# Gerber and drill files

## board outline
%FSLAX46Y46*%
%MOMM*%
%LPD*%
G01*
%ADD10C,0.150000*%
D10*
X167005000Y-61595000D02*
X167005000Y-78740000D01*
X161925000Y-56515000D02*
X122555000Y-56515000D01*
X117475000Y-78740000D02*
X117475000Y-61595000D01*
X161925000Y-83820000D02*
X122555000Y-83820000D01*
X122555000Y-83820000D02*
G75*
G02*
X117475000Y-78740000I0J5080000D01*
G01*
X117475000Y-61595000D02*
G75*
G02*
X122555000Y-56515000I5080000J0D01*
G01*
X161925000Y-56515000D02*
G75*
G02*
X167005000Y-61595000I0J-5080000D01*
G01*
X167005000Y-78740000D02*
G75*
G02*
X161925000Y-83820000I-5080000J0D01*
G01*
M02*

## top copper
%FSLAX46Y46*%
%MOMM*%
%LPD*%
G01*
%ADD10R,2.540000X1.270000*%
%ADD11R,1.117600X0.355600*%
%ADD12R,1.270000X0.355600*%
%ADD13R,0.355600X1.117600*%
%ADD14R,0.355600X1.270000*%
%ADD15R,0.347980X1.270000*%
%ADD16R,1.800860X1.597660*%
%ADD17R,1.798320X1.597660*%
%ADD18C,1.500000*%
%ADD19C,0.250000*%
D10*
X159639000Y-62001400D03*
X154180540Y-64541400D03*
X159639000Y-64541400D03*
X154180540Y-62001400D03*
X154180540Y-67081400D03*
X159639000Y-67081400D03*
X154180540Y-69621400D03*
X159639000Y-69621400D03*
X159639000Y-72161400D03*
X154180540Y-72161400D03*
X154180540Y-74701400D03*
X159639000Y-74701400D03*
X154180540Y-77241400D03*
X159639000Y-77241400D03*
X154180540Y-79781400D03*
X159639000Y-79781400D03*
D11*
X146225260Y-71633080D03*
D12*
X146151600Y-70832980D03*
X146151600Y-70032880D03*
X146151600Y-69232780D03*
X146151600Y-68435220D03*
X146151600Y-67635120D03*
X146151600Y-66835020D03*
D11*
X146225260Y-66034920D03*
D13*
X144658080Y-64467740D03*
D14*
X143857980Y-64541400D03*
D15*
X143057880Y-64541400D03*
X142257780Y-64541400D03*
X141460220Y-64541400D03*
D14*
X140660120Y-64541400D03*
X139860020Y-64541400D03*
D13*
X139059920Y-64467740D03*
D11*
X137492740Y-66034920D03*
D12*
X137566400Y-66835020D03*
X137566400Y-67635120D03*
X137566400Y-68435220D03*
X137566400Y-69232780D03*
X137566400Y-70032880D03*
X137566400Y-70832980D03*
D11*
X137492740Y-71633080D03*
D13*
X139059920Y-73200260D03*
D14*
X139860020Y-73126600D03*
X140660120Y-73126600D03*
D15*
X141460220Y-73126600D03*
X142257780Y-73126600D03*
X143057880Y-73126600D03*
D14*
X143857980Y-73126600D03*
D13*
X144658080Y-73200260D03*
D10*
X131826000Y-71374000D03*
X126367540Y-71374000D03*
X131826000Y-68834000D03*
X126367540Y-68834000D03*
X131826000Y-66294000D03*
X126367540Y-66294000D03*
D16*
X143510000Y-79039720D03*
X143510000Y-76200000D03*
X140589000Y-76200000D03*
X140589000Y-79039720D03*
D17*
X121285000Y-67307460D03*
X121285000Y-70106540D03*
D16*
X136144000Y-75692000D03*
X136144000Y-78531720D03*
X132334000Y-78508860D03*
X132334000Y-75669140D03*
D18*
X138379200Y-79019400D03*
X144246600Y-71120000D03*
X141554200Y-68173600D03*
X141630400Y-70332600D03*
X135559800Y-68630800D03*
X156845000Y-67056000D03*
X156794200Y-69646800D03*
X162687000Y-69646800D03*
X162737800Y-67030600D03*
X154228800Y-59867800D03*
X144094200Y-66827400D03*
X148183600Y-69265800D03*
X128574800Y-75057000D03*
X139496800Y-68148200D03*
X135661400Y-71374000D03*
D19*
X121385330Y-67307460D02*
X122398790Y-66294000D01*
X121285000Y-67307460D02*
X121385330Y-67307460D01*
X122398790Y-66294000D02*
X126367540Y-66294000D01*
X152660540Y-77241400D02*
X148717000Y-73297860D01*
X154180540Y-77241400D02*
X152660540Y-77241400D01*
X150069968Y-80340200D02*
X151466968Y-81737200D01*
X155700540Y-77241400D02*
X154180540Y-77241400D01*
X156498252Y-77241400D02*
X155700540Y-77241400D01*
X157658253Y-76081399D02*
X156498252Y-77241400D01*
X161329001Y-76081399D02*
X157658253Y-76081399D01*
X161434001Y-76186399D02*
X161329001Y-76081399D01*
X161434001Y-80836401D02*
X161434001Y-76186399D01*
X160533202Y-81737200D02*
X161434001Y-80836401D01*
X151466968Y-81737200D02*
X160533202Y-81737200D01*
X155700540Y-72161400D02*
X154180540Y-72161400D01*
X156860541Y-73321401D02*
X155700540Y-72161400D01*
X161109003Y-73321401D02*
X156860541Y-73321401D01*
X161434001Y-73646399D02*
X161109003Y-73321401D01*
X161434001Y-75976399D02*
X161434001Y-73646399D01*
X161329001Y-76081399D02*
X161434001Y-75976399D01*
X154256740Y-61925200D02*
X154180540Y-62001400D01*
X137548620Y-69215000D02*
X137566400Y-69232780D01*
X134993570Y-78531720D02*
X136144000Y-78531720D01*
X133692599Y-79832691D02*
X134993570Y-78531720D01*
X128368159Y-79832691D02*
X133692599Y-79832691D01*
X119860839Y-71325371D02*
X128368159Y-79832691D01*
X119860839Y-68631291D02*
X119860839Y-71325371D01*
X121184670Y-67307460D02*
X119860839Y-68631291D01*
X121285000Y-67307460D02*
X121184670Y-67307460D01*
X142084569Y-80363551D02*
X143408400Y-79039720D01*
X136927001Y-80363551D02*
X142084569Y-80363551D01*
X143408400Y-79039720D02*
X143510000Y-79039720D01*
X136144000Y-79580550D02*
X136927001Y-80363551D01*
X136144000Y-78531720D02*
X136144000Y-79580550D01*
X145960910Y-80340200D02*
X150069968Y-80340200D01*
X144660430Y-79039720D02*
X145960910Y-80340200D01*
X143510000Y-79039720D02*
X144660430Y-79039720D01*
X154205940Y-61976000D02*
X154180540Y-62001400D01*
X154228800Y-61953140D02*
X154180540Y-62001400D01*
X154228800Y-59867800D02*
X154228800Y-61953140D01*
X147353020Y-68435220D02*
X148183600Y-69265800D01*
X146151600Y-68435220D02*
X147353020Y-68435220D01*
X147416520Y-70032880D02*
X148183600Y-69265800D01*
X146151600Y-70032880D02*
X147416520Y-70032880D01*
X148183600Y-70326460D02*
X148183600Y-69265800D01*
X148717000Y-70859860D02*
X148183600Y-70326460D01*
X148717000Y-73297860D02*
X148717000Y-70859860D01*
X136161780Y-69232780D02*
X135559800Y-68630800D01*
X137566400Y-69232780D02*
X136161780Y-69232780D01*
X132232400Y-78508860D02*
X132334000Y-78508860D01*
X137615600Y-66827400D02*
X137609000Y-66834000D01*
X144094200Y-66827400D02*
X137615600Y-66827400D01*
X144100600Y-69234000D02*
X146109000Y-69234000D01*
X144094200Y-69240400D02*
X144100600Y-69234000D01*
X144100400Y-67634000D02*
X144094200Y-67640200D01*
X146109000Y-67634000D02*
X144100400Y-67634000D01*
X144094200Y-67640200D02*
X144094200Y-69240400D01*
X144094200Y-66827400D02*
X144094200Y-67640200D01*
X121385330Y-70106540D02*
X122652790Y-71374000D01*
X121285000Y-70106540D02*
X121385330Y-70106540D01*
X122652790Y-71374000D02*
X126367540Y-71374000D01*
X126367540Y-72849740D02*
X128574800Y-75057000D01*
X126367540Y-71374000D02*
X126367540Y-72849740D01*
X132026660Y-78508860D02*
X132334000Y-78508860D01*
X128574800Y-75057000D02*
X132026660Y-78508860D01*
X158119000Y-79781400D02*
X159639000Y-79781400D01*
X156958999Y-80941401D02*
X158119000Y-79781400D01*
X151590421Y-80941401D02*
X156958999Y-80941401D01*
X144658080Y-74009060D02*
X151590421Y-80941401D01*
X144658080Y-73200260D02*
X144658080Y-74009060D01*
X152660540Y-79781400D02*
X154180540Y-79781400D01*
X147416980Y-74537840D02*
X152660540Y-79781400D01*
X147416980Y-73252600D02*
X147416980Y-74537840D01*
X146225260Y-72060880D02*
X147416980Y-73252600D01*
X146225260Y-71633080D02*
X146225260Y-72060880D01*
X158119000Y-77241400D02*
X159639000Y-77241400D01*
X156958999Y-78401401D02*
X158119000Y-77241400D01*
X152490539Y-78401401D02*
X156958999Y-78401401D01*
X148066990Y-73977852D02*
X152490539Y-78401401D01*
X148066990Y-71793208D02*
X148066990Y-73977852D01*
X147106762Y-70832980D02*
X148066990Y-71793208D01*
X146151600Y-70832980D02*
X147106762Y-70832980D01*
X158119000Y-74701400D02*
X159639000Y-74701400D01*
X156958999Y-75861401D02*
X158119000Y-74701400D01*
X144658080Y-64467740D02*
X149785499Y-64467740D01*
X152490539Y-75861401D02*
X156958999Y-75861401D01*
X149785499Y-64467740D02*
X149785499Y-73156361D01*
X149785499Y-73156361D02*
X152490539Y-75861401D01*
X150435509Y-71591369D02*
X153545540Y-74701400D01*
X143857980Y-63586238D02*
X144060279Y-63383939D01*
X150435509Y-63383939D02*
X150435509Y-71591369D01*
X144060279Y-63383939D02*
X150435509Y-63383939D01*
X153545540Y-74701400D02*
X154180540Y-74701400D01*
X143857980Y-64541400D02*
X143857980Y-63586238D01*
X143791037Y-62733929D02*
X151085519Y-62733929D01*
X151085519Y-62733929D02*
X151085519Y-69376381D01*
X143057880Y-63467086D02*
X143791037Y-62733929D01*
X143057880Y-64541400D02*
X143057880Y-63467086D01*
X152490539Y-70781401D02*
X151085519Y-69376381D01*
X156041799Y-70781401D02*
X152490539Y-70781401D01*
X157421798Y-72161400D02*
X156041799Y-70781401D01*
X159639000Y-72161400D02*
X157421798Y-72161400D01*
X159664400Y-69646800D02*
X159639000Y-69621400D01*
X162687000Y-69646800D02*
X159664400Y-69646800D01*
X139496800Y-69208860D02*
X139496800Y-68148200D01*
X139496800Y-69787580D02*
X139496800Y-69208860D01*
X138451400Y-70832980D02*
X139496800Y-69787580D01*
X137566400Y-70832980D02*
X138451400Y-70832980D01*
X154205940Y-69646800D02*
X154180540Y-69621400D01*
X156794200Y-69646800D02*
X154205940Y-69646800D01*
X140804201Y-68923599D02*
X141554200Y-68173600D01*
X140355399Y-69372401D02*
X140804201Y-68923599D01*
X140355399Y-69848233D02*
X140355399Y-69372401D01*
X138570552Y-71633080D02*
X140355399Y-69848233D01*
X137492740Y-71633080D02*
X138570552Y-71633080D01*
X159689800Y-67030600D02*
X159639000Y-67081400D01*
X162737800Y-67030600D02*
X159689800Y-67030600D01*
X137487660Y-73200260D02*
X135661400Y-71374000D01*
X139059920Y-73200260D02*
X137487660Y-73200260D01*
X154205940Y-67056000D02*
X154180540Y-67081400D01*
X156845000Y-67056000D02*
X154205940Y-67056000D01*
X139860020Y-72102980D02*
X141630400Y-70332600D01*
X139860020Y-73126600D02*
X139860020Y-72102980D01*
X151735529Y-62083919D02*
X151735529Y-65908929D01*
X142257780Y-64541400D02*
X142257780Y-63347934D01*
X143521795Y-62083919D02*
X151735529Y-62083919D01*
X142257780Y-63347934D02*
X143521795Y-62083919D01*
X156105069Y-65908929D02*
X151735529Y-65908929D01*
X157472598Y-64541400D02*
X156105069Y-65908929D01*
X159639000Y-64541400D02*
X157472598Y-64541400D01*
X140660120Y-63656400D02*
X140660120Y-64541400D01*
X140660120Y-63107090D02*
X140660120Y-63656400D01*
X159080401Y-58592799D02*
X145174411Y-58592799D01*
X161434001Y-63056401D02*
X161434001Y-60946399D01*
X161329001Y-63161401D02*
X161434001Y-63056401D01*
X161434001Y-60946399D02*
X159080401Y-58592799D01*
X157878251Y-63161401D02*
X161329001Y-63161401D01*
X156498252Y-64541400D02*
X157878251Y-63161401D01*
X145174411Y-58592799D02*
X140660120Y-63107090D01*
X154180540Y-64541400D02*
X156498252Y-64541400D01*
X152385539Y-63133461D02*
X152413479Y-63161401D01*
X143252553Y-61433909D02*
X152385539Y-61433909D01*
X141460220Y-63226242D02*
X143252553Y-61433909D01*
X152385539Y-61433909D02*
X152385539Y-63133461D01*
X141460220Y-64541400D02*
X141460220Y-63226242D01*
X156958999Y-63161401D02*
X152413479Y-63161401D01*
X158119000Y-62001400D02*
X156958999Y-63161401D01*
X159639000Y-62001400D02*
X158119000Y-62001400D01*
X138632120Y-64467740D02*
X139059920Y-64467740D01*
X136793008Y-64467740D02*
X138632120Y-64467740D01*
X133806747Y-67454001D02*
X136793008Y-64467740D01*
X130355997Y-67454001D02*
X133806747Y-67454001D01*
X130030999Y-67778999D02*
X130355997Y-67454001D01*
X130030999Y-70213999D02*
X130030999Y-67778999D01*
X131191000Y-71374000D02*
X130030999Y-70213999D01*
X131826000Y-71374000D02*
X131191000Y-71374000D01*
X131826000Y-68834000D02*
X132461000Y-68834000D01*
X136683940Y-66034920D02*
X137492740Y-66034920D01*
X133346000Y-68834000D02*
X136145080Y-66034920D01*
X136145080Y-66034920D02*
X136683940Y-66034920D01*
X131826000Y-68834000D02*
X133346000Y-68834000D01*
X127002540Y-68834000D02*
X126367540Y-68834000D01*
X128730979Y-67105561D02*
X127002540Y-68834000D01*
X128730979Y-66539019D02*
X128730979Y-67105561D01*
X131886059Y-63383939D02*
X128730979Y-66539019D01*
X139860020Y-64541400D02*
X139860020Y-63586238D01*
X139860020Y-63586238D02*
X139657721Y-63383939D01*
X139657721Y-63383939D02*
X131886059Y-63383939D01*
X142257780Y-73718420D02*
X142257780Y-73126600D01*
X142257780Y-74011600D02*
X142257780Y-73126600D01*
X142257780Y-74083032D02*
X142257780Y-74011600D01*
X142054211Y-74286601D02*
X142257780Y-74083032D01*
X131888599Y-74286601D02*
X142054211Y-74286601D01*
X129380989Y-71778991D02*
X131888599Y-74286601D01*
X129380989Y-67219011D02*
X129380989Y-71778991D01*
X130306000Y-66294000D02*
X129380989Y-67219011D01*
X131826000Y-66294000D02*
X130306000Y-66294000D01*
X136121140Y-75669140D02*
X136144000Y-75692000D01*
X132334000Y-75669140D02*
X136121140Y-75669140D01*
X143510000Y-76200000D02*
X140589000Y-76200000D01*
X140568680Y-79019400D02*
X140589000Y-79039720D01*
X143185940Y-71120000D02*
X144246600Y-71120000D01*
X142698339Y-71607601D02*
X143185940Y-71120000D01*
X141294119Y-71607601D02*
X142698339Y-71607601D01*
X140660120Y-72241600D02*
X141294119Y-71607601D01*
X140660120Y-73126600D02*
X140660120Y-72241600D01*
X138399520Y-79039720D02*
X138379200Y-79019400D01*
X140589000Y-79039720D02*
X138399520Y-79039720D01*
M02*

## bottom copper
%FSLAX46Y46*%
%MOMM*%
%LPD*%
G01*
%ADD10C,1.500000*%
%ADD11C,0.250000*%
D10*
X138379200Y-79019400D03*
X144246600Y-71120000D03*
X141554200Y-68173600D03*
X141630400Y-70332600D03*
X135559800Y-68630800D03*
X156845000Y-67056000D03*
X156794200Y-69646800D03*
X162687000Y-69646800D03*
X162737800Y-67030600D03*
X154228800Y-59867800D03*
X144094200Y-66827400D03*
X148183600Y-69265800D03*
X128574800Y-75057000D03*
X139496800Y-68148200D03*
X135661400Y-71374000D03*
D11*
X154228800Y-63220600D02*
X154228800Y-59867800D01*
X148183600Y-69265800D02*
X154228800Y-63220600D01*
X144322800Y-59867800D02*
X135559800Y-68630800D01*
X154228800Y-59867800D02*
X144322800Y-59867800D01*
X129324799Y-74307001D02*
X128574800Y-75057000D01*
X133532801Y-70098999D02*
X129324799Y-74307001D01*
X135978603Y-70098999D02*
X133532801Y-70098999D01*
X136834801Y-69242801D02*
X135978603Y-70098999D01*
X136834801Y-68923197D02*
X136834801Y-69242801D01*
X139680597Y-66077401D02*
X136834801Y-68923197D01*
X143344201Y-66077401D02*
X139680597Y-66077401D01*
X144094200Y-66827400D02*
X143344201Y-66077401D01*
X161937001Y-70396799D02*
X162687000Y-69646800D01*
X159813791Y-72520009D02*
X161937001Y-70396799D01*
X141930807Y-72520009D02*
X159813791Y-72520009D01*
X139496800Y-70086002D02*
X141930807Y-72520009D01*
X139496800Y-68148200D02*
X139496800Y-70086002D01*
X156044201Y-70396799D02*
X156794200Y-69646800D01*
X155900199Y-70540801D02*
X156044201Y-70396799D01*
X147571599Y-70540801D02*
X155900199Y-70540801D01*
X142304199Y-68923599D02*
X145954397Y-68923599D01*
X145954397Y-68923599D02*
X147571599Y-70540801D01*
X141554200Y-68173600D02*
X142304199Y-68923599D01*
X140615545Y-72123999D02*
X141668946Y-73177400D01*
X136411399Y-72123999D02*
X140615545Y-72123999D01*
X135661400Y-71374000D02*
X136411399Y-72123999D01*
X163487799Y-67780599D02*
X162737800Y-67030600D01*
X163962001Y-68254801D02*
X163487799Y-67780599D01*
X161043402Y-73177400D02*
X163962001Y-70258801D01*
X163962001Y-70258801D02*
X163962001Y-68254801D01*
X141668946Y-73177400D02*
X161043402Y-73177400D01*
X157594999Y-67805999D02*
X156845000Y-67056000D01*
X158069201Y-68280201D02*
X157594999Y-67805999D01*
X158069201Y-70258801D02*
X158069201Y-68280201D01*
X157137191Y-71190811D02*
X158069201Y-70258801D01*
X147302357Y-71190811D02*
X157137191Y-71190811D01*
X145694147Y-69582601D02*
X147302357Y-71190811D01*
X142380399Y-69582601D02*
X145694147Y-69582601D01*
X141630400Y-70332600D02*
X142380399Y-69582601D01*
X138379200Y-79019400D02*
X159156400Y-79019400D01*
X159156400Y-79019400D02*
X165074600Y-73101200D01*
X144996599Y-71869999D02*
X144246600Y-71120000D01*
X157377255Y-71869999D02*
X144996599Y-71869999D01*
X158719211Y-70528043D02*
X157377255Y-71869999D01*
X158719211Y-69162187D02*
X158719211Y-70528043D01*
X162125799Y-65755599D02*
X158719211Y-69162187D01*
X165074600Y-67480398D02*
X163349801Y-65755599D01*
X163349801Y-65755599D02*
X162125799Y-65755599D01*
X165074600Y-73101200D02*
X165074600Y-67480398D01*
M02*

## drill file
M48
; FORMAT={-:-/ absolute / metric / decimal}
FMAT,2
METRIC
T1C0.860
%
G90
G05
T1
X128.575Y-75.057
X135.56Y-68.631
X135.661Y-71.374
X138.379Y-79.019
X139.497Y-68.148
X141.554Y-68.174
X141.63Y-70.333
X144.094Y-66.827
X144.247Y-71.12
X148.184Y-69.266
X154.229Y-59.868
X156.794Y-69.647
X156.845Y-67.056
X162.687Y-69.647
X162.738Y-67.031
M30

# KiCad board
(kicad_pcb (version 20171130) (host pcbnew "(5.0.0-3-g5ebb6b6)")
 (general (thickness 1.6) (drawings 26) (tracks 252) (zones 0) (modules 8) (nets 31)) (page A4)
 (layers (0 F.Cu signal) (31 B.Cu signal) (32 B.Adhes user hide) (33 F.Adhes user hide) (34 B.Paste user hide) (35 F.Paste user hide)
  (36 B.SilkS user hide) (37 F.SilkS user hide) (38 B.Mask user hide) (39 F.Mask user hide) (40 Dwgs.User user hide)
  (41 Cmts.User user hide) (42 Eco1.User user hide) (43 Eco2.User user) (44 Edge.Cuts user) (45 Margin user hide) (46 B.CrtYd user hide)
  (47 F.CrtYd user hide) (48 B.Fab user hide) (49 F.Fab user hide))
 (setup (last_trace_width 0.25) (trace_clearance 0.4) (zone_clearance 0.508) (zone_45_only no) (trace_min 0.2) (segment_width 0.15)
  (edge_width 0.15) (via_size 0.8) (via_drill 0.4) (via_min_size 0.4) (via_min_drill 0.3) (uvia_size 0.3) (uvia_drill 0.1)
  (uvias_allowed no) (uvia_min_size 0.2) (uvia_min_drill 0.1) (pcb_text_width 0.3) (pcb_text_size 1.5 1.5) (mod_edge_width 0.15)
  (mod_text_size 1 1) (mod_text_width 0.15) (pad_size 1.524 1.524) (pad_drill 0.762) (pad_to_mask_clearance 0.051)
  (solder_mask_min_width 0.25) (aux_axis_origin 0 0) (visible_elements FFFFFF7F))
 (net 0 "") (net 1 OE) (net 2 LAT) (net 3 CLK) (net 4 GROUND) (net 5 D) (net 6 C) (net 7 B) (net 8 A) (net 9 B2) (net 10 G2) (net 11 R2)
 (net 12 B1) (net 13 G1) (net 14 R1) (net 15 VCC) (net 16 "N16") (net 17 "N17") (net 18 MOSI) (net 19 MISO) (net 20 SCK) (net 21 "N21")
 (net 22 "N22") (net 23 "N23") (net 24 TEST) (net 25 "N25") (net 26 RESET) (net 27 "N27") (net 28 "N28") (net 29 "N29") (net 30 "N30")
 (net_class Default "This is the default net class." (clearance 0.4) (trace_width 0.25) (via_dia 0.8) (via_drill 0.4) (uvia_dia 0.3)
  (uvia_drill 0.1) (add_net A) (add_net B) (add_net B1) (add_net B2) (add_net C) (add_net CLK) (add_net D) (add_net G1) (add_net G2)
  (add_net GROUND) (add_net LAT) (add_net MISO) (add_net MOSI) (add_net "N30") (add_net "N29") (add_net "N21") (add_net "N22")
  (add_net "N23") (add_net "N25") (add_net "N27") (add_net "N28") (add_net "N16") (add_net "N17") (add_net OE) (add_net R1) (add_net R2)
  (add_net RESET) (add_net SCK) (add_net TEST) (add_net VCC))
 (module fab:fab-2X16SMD (layer F.Cu) (at 157.099 77.2414 180)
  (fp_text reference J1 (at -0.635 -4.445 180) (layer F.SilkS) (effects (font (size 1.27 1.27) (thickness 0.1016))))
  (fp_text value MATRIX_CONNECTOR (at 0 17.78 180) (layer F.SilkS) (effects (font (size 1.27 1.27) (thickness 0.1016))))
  (pad 15 smd rect (at -2.54 15.24 180) (size 2.54 1.27) (layers F.Cu F.Paste F.Mask) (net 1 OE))
  (pad 14 smd rect (at 2.91846 12.7 180) (size 2.54 1.27) (layers F.Cu F.Paste F.Mask) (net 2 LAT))
  (pad 13 smd rect (at -2.54 12.7 180) (size 2.54 1.27) (layers F.Cu F.Paste F.Mask) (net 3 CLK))
  (pad 16 smd rect (at 2.91846 15.24 180) (size 2.54 1.27) (layers F.Cu F.Paste F.Mask) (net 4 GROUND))
  (pad 12 smd rect (at 2.91846 10.16 180) (size 2.54 1.27) (layers F.Cu F.Paste F.Mask) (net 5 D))
  (pad 11 smd rect (at -2.54 10.16 180) (size 2.54 1.27) (layers F.Cu F.Paste F.Mask) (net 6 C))
  (pad 10 smd rect (at 2.91846 7.62 180) (size 2.54 1.27) (layers F.Cu F.Paste F.Mask) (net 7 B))
  (pad 9 smd rect (at -2.54 7.62 180) (size 2.54 1.27) (layers F.Cu F.Paste F.Mask) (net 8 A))
  (pad 7 smd rect (at -2.54 5.08 180) (size 2.54 1.27) (layers F.Cu F.Paste F.Mask) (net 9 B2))
  (pad 8 smd rect (at 2.91846 5.08 180) (size 2.54 1.27) (layers F.Cu F.Paste F.Mask) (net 4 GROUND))
  (pad 6 smd rect (at 2.91846 2.54 180) (size 2.54 1.27) (layers F.Cu F.Paste F.Mask) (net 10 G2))
  (pad 5 smd rect (at -2.54 2.54 180) (size 2.54 1.27) (layers F.Cu F.Paste F.Mask) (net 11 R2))
  (pad 4 smd rect (at 2.91846 0 180) (size 2.54 1.27) (layers F.Cu F.Paste F.Mask) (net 4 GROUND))
  (pad 3 smd rect (at -2.54 0 180) (size 2.54 1.27) (layers F.Cu F.Paste F.Mask) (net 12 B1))
  (pad 2 smd rect (at 2.91846 -2.54 180) (size 2.54 1.27) (layers F.Cu F.Paste F.Mask) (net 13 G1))
  (pad 1 smd rect (at -2.54 -2.54 180) (size 2.54 1.27) (layers F.Cu F.Paste F.Mask) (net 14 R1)))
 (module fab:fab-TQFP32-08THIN (layer F.Cu) (at 141.859 68.834 180)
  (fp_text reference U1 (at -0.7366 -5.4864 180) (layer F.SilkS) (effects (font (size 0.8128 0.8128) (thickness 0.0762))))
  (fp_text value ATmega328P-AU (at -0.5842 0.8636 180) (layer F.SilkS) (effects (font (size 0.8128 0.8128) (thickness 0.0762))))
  (pad 1 smd rect (at -4.36626 -2.79908 180) (size 1.1176 0.3556) (layers F.Cu F.Paste F.Mask) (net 13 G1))
  (pad 2 smd rect (at -4.2926 -1.99898 180) (size 1.27 0.3556) (layers F.Cu F.Paste F.Mask) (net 12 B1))
  (pad 3 smd rect (at -4.2926 -1.19888 180) (size 1.27 0.3556) (layers F.Cu F.Paste F.Mask) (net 4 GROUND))
  (pad 4 smd rect (at -4.2926 -0.39878 180) (size 1.27 0.3556) (layers F.Cu F.Paste F.Mask) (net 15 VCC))
  (pad 5 smd rect (at -4.2926 0.39878 180) (size 1.27 0.3556) (layers F.Cu F.Paste F.Mask) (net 4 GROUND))
  (pad 6 smd rect (at -4.2926 1.19888 180) (size 1.27 0.3556) (layers F.Cu F.Paste F.Mask) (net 15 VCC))
  (pad 7 smd rect (at -4.2926 1.99898 180) (size 1.27 0.3556) (layers F.Cu F.Paste F.Mask) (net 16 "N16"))
  (pad 8 smd rect (at -4.36626 2.79908 180) (size 1.1176 0.3556) (layers F.Cu F.Paste F.Mask) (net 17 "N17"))
  (pad 9 smd rect (at -2.79908 4.36626 180) (size 0.3556 1.1176) (layers F.Cu F.Paste F.Mask) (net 11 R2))
  (pad 10 smd rect (at -1.99898 4.2926 180) (size 0.3556 1.27) (layers F.Cu F.Paste F.Mask) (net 10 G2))
  (pad 11 smd rect (at -1.19888 4.2926 180) (size 0.34798 1.27) (layers F.Cu F.Paste F.Mask) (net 9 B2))
  (pad 12 smd rect (at -0.39878 4.2926 180) (size 0.34798 1.27) (layers F.Cu F.Paste F.Mask) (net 3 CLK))
  (pad 13 smd rect (at 0.39878 4.2926 180) (size 0.34798 1.27) (layers F.Cu F.Paste F.Mask) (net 1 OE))
  (pad 14 smd rect (at 1.19888 4.2926 180) (size 0.3556 1.27) (layers F.Cu F.Paste F.Mask) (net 2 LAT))
  (pad 15 smd rect (at 1.99898 4.2926 180) (size 0.3556 1.27) (layers F.Cu F.Paste F.Mask) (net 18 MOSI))
  (pad 16 smd rect (at 2.79908 4.36626 180) (size 0.3556 1.1176) (layers F.Cu F.Paste F.Mask) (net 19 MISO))
  (pad 17 smd rect (at 4.36626 2.79908 180) (size 1.1176 0.3556) (layers F.Cu F.Paste F.Mask) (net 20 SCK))
  (pad 18 smd rect (at 4.2926 1.99898 180) (size 1.27 0.3556) (layers F.Cu F.Paste F.Mask) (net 15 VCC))
  (pad 19 smd rect (at 4.2926 1.19888 180) (size 1.27 0.3556) (layers F.Cu F.Paste F.Mask) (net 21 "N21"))
  (pad 20 smd rect (at 4.2926 0.39878 180) (size 1.27 0.3556) (layers F.Cu F.Paste F.Mask) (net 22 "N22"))
  (pad 21 smd rect (at 4.2926 -0.39878 180) (size 1.27 0.3556) (layers F.Cu F.Paste F.Mask) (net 4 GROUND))
  (pad 22 smd rect (at 4.2926 -1.19888 180) (size 1.27 0.3556) (layers F.Cu F.Paste F.Mask) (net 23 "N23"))
  (pad 23 smd rect (at 4.2926 -1.99898 180) (size 1.27 0.3556) (layers F.Cu F.Paste F.Mask) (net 8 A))
  (pad 24 smd rect (at 4.36626 -2.79908 180) (size 1.1176 0.3556) (layers F.Cu F.Paste F.Mask) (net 7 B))
  (pad 25 smd rect (at 2.79908 -4.36626 180) (size 0.3556 1.1176) (layers F.Cu F.Paste F.Mask) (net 6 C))
  (pad 26 smd rect (at 1.99898 -4.2926 180) (size 0.3556 1.27) (layers F.Cu F.Paste F.Mask) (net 5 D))
  (pad 27 smd rect (at 1.19888 -4.2926 180) (size 0.3556 1.27) (layers F.Cu F.Paste F.Mask) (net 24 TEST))
  (pad 28 smd rect (at 0.39878 -4.2926 180) (size 0.34798 1.27) (layers F.Cu F.Paste F.Mask) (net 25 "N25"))
  (pad 29 smd rect (at -0.39878 -4.2926 180) (size 0.34798 1.27) (layers F.Cu F.Paste F.Mask) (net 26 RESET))
  (pad 30 smd rect (at -1.19888 -4.2926 180) (size 0.34798 1.27) (layers F.Cu F.Paste F.Mask) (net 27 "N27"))
  (pad 31 smd rect (at -1.99898 -4.2926 180) (size 0.3556 1.27) (layers F.Cu F.Paste F.Mask) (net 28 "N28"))
  (pad 32 smd rect (at -2.79908 -4.36626 180) (size 0.3556 1.1176) (layers F.Cu F.Paste F.Mask) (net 14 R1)))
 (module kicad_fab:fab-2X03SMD (layer F.Cu) (at 129.286 68.834 180)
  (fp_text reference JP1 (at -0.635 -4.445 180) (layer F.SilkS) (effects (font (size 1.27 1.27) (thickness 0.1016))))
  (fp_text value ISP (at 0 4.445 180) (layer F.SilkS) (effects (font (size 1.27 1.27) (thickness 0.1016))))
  (pad 1 smd rect (at -2.54 -2.54 180) (size 2.54 1.27) (layers F.Cu F.Paste F.Mask) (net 19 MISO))
  (pad 2 smd rect (at 2.91846 -2.54 180) (size 2.54 1.27) (layers F.Cu F.Paste F.Mask) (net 15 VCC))
  (pad 3 smd rect (at -2.54 0 180) (size 2.54 1.27) (layers F.Cu F.Paste F.Mask) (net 20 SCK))
  (pad 4 smd rect (at 2.91846 0 180) (size 2.54 1.27) (layers F.Cu F.Paste F.Mask) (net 18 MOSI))
  (pad 5 smd rect (at -2.54 2.54 180) (size 2.54 1.27) (layers F.Cu F.Paste F.Mask) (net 26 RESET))
  (pad 6 smd rect (at 2.91846 2.54 180) (size 2.54 1.27) (layers F.Cu F.Paste F.Mask) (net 4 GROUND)))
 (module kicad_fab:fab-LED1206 (layer F.Cu) (at 143.51 77.61986 270)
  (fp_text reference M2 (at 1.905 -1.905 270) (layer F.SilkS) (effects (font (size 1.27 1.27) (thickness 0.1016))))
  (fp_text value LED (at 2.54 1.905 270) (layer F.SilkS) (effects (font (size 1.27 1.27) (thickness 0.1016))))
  (pad 2 smd rect (at 1.41986 0 270) (size 1.59766 1.80086) (layers F.Cu F.Paste F.Mask) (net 4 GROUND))
  (pad 1 smd rect (at -1.41986 0 270) (size 1.59766 1.80086) (layers F.Cu F.Paste F.Mask) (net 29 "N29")))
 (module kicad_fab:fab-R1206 (layer F.Cu) (at 140.589 77.61986 90)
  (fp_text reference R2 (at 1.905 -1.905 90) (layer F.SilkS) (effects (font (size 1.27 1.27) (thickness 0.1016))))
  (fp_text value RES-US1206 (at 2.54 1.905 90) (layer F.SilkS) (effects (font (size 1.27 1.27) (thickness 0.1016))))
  (pad 2 smd rect (at 1.41986 0 90) (size 1.59766 1.80086) (layers F.Cu F.Paste F.Mask) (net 29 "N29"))
  (pad 1 smd rect (at -1.41986 0 90) (size 1.59766 1.80086) (layers F.Cu F.Paste F.Mask) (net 24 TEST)))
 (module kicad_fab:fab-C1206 (layer F.Cu) (at 121.285 68.707 270)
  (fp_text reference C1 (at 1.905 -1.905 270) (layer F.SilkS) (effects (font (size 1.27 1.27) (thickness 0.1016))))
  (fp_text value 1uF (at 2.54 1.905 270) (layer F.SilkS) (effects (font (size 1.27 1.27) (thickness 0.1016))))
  (pad 1 smd rect (at -1.39954 0 270) (size 1.59766 1.79832) (layers F.Cu F.Paste F.Mask) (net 4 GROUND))
  (pad 2 smd rect (at 1.39954 0 270) (size 1.59766 1.79832) (layers F.Cu F.Paste F.Mask) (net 15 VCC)))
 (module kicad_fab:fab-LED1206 (layer F.Cu) (at 136.144 77.11186 270)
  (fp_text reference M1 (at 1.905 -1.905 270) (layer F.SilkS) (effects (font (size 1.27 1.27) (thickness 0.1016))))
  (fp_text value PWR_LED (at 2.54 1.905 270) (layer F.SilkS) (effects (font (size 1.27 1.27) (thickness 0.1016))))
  (pad 1 smd rect (at -1.41986 0 270) (size 1.59766 1.80086) (layers F.Cu F.Paste F.Mask) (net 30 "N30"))
  (pad 2 smd rect (at 1.41986 0 270) (size 1.59766 1.80086) (layers F.Cu F.Paste F.Mask) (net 4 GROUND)))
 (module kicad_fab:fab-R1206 (layer F.Cu) (at 132.334 77.089 90)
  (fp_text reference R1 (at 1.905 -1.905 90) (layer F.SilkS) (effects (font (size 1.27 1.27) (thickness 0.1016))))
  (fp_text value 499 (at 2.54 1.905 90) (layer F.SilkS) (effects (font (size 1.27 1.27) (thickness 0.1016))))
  (pad 1 smd rect (at -1.41986 0 90) (size 1.59766 1.80086) (layers F.Cu F.Paste F.Mask) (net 15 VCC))
  (pad 2 smd rect (at 1.41986 0 90) (size 1.59766 1.80086) (layers F.Cu F.Paste F.Mask) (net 30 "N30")))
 (gr_line (start 167.005 61.595) (end 167.005 78.74) (layer Edge.Cuts) (width 0.15))
 (gr_line (start 161.925 56.515) (end 122.555 56.515) (layer Edge.Cuts) (width 0.15))
 (gr_line (start 117.475 78.74) (end 117.475 61.595) (layer Edge.Cuts) (width 0.15))
 (gr_line (start 161.925 83.82) (end 122.555 83.82) (layer Edge.Cuts) (width 0.15))
 (gr_arc (start 122.555 78.74) (end 117.475 78.74) (angle -90) (layer Edge.Cuts) (width 0.15))
 (gr_arc (start 122.555 61.595) (end 122.555 56.515) (angle -90) (layer Edge.Cuts) (width 0.15))
 (gr_arc (start 161.925 61.595) (end 167.005 61.595) (angle -90) (layer Edge.Cuts) (width 0.15))
 (gr_arc (start 161.925 78.74) (end 161.925 83.82) (angle -90) (layer Edge.Cuts) (width 0.15))
 (via (at 138.3792 79.0194) (size 1.5) (drill 0.86) (layers F.Cu B.Cu) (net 24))
 (via (at 144.2466 71.12) (size 1.5) (drill 0.86) (layers F.Cu B.Cu) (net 24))
 (via (at 141.5542 68.1736) (size 1.5) (drill 0.86) (layers F.Cu B.Cu) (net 7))
 (via (at 141.6304 70.3326) (size 1.5) (drill 0.86) (layers F.Cu B.Cu) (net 5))
 (via (at 135.5598 68.6308) (size 1.5) (drill 0.86) (layers F.Cu B.Cu) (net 4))
 (via (at 156.845 67.056) (size 1.5) (drill 0.86) (layers F.Cu B.Cu) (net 5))
 (via (at 156.7942 69.6468) (size 1.5) (drill 0.86) (layers F.Cu B.Cu) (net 7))
 (via (at 162.687 69.6468) (size 1.5) (drill 0.86) (layers F.Cu B.Cu) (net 8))
 (via (at 162.7378 67.0306) (size 1.5) (drill 0.86) (layers F.Cu B.Cu) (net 6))
 (via (at 154.2288 59.8678) (size 1.5) (drill 0.86) (layers F.Cu B.Cu) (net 4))
 (via (at 144.0942 66.8274) (size 1.5) (drill 0.86) (layers F.Cu B.Cu) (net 15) (status 1000000))
 (segment (start 121.38533 67.30746) (end 122.39879 66.294) (width 0.25) (layer F.Cu) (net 4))
 (segment (start 121.285 67.30746) (end 121.38533 67.30746) (width 0.25) (layer F.Cu) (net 4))
 (segment (start 122.39879 66.294) (end 126.36754 66.294) (width 0.25) (layer F.Cu) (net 4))
 (segment (start 152.66054 77.2414) (end 148.717 73.29786) (width 0.25) (layer F.Cu) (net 4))
 (segment (start 154.18054 77.2414) (end 152.66054 77.2414) (width 0.25) (layer F.Cu) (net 4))
 (segment (start 150.069968 80.3402) (end 151.466968 81.7372) (width 0.25) (layer F.Cu) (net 4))
 (segment (start 155.70054 77.2414) (end 154.18054 77.2414) (width 0.25) (layer F.Cu) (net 4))
 (segment (start 156.498252 77.2414) (end 155.70054 77.2414) (width 0.25) (layer F.Cu) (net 4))
 (segment (start 157.658253 76.081399) (end 156.498252 77.2414) (width 0.25) (layer F.Cu) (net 4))
 (segment (start 161.329001 76.081399) (end 157.658253 76.081399) (width 0.25) (layer F.Cu) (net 4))
 (segment (start 161.434001 76.186399) (end 161.329001 76.081399) (width 0.25) (layer F.Cu) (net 4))
 (segment (start 161.434001 80.836401) (end 161.434001 76.186399) (width 0.25) (layer F.Cu) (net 4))
 (segment (start 160.533202 81.7372) (end 161.434001 80.836401) (width 0.25) (layer F.Cu) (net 4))
 (segment (start 151.466968 81.7372) (end 160.533202 81.7372) (width 0.25) (layer F.Cu) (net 4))
 (segment (start 155.70054 72.1614) (end 154.18054 72.1614) (width 0.25) (layer F.Cu) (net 4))
 (segment (start 156.860541 73.321401) (end 155.70054 72.1614) (width 0.25) (layer F.Cu) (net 4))
 (segment (start 161.109003 73.321401) (end 156.860541 73.321401) (width 0.25) (layer F.Cu) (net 4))
 (segment (start 161.434001 73.646399) (end 161.109003 73.321401) (width 0.25) (layer F.Cu) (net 4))
 (segment (start 161.434001 75.976399) (end 161.434001 73.646399) (width 0.25) (layer F.Cu) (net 4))
 (segment (start 161.329001 76.081399) (end 161.434001 75.976399) (width 0.25) (layer F.Cu) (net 4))
 (segment (start 154.25674 61.9252) (end 154.18054 62.0014) (width 0.25) (layer F.Cu) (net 4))
 (segment (start 137.54862 69.215) (end 137.5664 69.23278) (width 0.25) (layer F.Cu) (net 4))
 (segment (start 134.99357 78.53172) (end 136.144 78.53172) (width 0.25) (layer F.Cu) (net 4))
 (segment (start 133.692599 79.832691) (end 134.99357 78.53172) (width 0.25) (layer F.Cu) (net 4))
 (segment (start 128.368159 79.832691) (end 133.692599 79.832691) (width 0.25) (layer F.Cu) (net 4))
 (segment (start 119.860839 71.325371) (end 128.368159 79.832691) (width 0.25) (layer F.Cu) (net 4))
 (segment (start 119.860839 68.631291) (end 119.860839 71.325371) (width 0.25) (layer F.Cu) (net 4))
 (segment (start 121.18467 67.30746) (end 119.860839 68.631291) (width 0.25) (layer F.Cu) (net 4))
 (segment (start 121.285 67.30746) (end 121.18467 67.30746) (width 0.25) (layer F.Cu) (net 4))
 (segment (start 142.084569 80.363551) (end 143.4084 79.03972) (width 0.25) (layer F.Cu) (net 4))
 (segment (start 136.927001 80.363551) (end 142.084569 80.363551) (width 0.25) (layer F.Cu) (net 4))
 (segment (start 143.4084 79.03972) (end 143.51 79.03972) (width 0.25) (layer F.Cu) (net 4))
 (segment (start 136.144 79.58055) (end 136.927001 80.363551) (width 0.25) (layer F.Cu) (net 4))
 (segment (start 136.144 78.53172) (end 136.144 79.58055) (width 0.25) (layer F.Cu) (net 4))
 (segment (start 145.96091 80.3402) (end 150.069968 80.3402) (width 0.25) (layer F.Cu) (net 4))
 (segment (start 144.66043 79.03972) (end 145.96091 80.3402) (width 0.25) (layer F.Cu) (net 4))
 (segment (start 143.51 79.03972) (end 144.66043 79.03972) (width 0.25) (layer F.Cu) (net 4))
 (segment (start 154.20594 61.976) (end 154.18054 62.0014) (width 0.25) (layer F.Cu) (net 4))
 (segment (start 154.2288 61.95314) (end 154.18054 62.0014) (width 0.25) (layer F.Cu) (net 4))
 (segment (start 154.2288 59.8678) (end 154.2288 61.95314) (width 0.25) (layer F.Cu) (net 4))
 (via (at 148.1836 69.2658) (size 1.5) (drill 0.86) (layers F.Cu B.Cu) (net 4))
 (segment (start 147.35302 68.43522) (end 148.1836 69.2658) (width 0.25) (layer F.Cu) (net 4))
 (segment (start 146.1516 68.43522) (end 147.35302 68.43522) (width 0.25) (layer F.Cu) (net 4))
 (segment (start 147.41652 70.03288) (end 148.1836 69.2658) (width 0.25) (layer F.Cu) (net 4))
 (segment (start 146.1516 70.03288) (end 147.41652 70.03288) (width 0.25) (layer F.Cu) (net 4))
 (segment (start 148.1836 70.32646) (end 148.1836 69.2658) (width 0.25) (layer F.Cu) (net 4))
 (segment (start 148.717 70.85986) (end 148.1836 70.32646) (width 0.25) (layer F.Cu) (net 4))
 (segment (start 148.717 73.29786) (end 148.717 70.85986) (width 0.25) (layer F.Cu) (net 4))
 (segment (start 154.2288 63.2206) (end 154.2288 59.8678) (width 0.25) (layer B.Cu) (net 4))
 (segment (start 148.1836 69.2658) (end 154.2288 63.2206) (width 0.25) (layer B.Cu) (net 4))
 (segment (start 136.16178 69.23278) (end 135.5598 68.6308) (width 0.25) (layer F.Cu) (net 4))
 (segment (start 137.5664 69.23278) (end 136.16178 69.23278) (width 0.25) (layer F.Cu) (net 4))
 (segment (start 144.3228 59.8678) (end 135.5598 68.6308) (width 0.25) (layer B.Cu) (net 4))
 (segment (start 154.2288 59.8678) (end 144.3228 59.8678) (width 0.25) (layer B.Cu) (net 4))
 (segment (start 132.2324 78.50886) (end 132.334 78.50886) (width 0.25) (layer F.Cu) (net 15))
 (segment (start 137.6156 66.8274) (end 137.609 66.834) (width 0.25) (layer F.Cu) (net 15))
 (segment (start 144.0942 66.8274) (end 137.6156 66.8274) (width 0.25) (layer F.Cu) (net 15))
 (segment (start 144.1006 69.234) (end 146.109 69.234) (width 0.25) (layer F.Cu) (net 15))
 (segment (start 144.0942 69.2404) (end 144.1006 69.234) (width 0.25) (layer F.Cu) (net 15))
 (segment (start 144.1004 67.634) (end 144.0942 67.6402) (width 0.25) (layer F.Cu) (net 15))
 (segment (start 146.109 67.634) (end 144.1004 67.634) (width 0.25) (layer F.Cu) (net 15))
 (segment (start 144.0942 67.6402) (end 144.0942 69.2404) (width 0.25) (layer F.Cu) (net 15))
 (segment (start 144.0942 66.8274) (end 144.0942 67.6402) (width 0.25) (layer F.Cu) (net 15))
 (segment (start 121.38533 70.10654) (end 122.65279 71.374) (width 0.25) (layer F.Cu) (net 15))
 (segment (start 121.285 70.10654) (end 121.38533 70.10654) (width 0.25) (layer F.Cu) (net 15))
 (segment (start 122.65279 71.374) (end 126.36754 71.374) (width 0.25) (layer F.Cu) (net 15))
 (via (at 128.5748 75.057) (size 1.5) (drill 0.86) (layers F.Cu B.Cu) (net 15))
 (segment (start 126.36754 72.84974) (end 128.5748 75.057) (width 0.25) (layer F.Cu) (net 15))
 (segment (start 126.36754 71.374) (end 126.36754 72.84974) (width 0.25) (layer F.Cu) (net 15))
 (segment (start 132.02666 78.50886) (end 132.334 78.50886) (width 0.25) (layer F.Cu) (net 15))
 (segment (start 128.5748 75.057) (end 132.02666 78.50886) (width 0.25) (layer F.Cu) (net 15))
 (segment (start 129.324799 74.307001) (end 128.5748 75.057) (width 0.25) (layer B.Cu) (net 15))
 (segment (start 133.532801 70.098999) (end 129.324799 74.307001) (width 0.25) (layer B.Cu) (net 15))
 (segment (start 135.978603 70.098999) (end 133.532801 70.098999) (width 0.25) (layer B.Cu) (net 15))
 (segment (start 136.834801 69.242801) (end 135.978603 70.098999) (width 0.25) (layer B.Cu) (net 15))
 (segment (start 136.834801 68.923197) (end 136.834801 69.242801) (width 0.25) (layer B.Cu) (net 15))
 (segment (start 139.680597 66.077401) (end 136.834801 68.923197) (width 0.25) (layer B.Cu) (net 15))
 (segment (start 143.344201 66.077401) (end 139.680597 66.077401) (width 0.25) (layer B.Cu) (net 15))
 (segment (start 144.0942 66.8274) (end 143.344201 66.077401) (width 0.25) (layer B.Cu) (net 15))
 (segment (start 158.119 79.7814) (end 159.639 79.7814) (width 0.25) (layer F.Cu) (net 14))
 (segment (start 156.958999 80.941401) (end 158.119 79.7814) (width 0.25) (layer F.Cu) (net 14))
 (segment (start 151.590421 80.941401) (end 156.958999 80.941401) (width 0.25) (layer F.Cu) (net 14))
 (segment (start 144.65808 74.00906) (end 151.590421 80.941401) (width 0.25) (layer F.Cu) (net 14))
 (segment (start 144.65808 73.20026) (end 144.65808 74.00906) (width 0.25) (layer F.Cu) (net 14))
 (segment (start 152.66054 79.7814) (end 154.18054 79.7814) (width 0.25) (layer F.Cu) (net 13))
 (segment (start 147.41698 74.53784) (end 152.66054 79.7814) (width 0.25) (layer F.Cu) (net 13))
 (segment (start 147.41698 73.2526) (end 147.41698 74.53784) (width 0.25) (layer F.Cu) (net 13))
 (segment (start 146.22526 72.06088) (end 147.41698 73.2526) (width 0.25) (layer F.Cu) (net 13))
 (segment (start 146.22526 71.63308) (end 146.22526 72.06088) (width 0.25) (layer F.Cu) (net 13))
 (segment (start 158.119 77.2414) (end 159.639 77.2414) (width 0.25) (layer F.Cu) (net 12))
 (segment (start 156.958999 78.401401) (end 158.119 77.2414) (width 0.25) (layer F.Cu) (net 12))
 (segment (start 152.490539 78.401401) (end 156.958999 78.401401) (width 0.25) (layer F.Cu) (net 12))
 (segment (start 148.06699 73.977852) (end 152.490539 78.401401) (width 0.25) (layer F.Cu) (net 12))
 (segment (start 148.06699 71.793208) (end 148.06699 73.977852) (width 0.25) (layer F.Cu) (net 12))
 (segment (start 147.106762 70.83298) (end 148.06699 71.793208) (width 0.25) (layer F.Cu) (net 12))
 (segment (start 146.1516 70.83298) (end 147.106762 70.83298) (width 0.25) (layer F.Cu) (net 12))
 (segment (start 158.119 74.7014) (end 159.639 74.7014) (width 0.25) (layer F.Cu) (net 11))
 (segment (start 156.958999 75.861401) (end 158.119 74.7014) (width 0.25) (layer F.Cu) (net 11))
 (segment (start 144.65808 64.46774) (end 149.785499 64.46774) (width 0.25) (layer F.Cu) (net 11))
 (segment (start 152.490539 75.861401) (end 156.958999 75.861401) (width 0.25) (layer F.Cu) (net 11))
 (segment (start 149.785499 64.46774) (end 149.785499 73.156361) (width 0.25) (layer F.Cu) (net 11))
 (segment (start 149.785499 73.156361) (end 152.490539 75.861401) (width 0.25) (layer F.Cu) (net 11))
 (segment (start 150.435509 71.591369) (end 153.54554 74.7014) (width 0.25) (layer F.Cu) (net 10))
 (segment (start 143.85798 63.586238) (end 144.060279 63.383939) (width 0.25) (layer F.Cu) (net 10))
 (segment (start 150.435509 63.383939) (end 150.435509 71.591369) (width 0.25) (layer F.Cu) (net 10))
 (segment (start 144.060279 63.383939) (end 150.435509 63.383939) (width 0.25) (layer F.Cu) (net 10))
 (segment (start 153.54554 74.7014) (end 154.18054 74.7014) (width 0.25) (layer F.Cu) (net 10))
 (segment (start 143.85798 64.5414) (end 143.85798 63.586238) (width 0.25) (layer F.Cu) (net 10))
 (segment (start 143.791037 62.733929) (end 151.085519 62.733929) (width 0.25) (layer F.Cu) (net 9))
 (segment (start 151.085519 62.733929) (end 151.085519 69.376381) (width 0.25) (layer F.Cu) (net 9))
 (segment (start 143.05788 63.467086) (end 143.791037 62.733929) (width 0.25) (layer F.Cu) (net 9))
 (segment (start 143.05788 64.5414) (end 143.05788 63.467086) (width 0.25) (layer F.Cu) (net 9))
 (segment (start 152.490539 70.781401) (end 151.085519 69.376381) (width 0.25) (layer F.Cu) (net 9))
 (segment (start 156.041799 70.781401) (end 152.490539 70.781401) (width 0.25) (layer F.Cu) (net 9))
 (segment (start 157.421798 72.1614) (end 156.041799 70.781401) (width 0.25) (layer F.Cu) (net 9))
 (segment (start 159.639 72.1614) (end 157.421798 72.1614) (width 0.25) (layer F.Cu) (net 9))
 (segment (start 159.6644 69.6468) (end 159.639 69.6214) (width 0.25) (layer F.Cu) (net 8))
 (segment (start 162.687 69.6468) (end 159.6644 69.6468) (width 0.25) (layer F.Cu) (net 8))
 (via (at 139.4968 68.1482) (size 1.5) (drill 0.86) (layers F.Cu B.Cu) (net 8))
 (segment (start 139.4968 69.20886) (end 139.4968 68.1482) (width 0.25) (layer F.Cu) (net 8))
 (segment (start 139.4968 69.78758) (end 139.4968 69.20886) (width 0.25) (layer F.Cu) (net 8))
 (segment (start 138.4514 70.83298) (end 139.4968 69.78758) (width 0.25) (layer F.Cu) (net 8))
 (segment (start 137.5664 70.83298) (end 138.4514 70.83298) (width 0.25) (layer F.Cu) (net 8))
 (segment (start 161.937001 70.396799) (end 162.687 69.6468) (width 0.25) (layer B.Cu) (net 8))
 (segment (start 159.813791 72.520009) (end 161.937001 70.396799) (width 0.25) (layer B.Cu) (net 8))
 (segment (start 141.930807 72.520009) (end 159.813791 72.520009) (width 0.25) (layer B.Cu) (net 8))
 (segment (start 139.4968 70.086002) (end 141.930807 72.520009) (width 0.25) (layer B.Cu) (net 8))
 (segment (start 139.4968 68.1482) (end 139.4968 70.086002) (width 0.25) (layer B.Cu) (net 8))
 (segment (start 154.20594 69.6468) (end 154.18054 69.6214) (width 0.25) (layer F.Cu) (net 7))
 (segment (start 156.7942 69.6468) (end 154.20594 69.6468) (width 0.25) (layer F.Cu) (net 7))
 (segment (start 140.804201 68.923599) (end 141.5542 68.1736) (width 0.25) (layer F.Cu) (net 7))
 (segment (start 140.355399 69.372401) (end 140.804201 68.923599) (width 0.25) (layer F.Cu) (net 7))
 (segment (start 140.355399 69.848233) (end 140.355399 69.372401) (width 0.25) (layer F.Cu) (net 7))
 (segment (start 138.570552 71.63308) (end 140.355399 69.848233) (width 0.25) (layer F.Cu) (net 7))
 (segment (start 137.49274 71.63308) (end 138.570552 71.63308) (width 0.25) (layer F.Cu) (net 7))
 (segment (start 156.044201 70.396799) (end 156.7942 69.6468) (width 0.25) (layer B.Cu) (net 7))
 (segment (start 155.900199 70.540801) (end 156.044201 70.396799) (width 0.25) (layer B.Cu) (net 7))
 (segment (start 147.571599 70.540801) (end 155.900199 70.540801) (width 0.25) (layer B.Cu) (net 7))
 (segment (start 142.304199 68.923599) (end 145.954397 68.923599) (width 0.25) (layer B.Cu) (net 7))
 (segment (start 145.954397 68.923599) (end 147.571599 70.540801) (width 0.25) (layer B.Cu) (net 7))
 (segment (start 141.5542 68.1736) (end 142.304199 68.923599) (width 0.25) (layer B.Cu) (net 7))
 (segment (start 159.6898 67.0306) (end 159.639 67.0814) (width 0.25) (layer F.Cu) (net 6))
 (segment (start 162.7378 67.0306) (end 159.6898 67.0306) (width 0.25) (layer F.Cu) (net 6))
 (via (at 135.6614 71.374) (size 1.5) (drill 0.86) (layers F.Cu B.Cu) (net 6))
 (segment (start 137.48766 73.20026) (end 135.6614 71.374) (width 0.25) (layer F.Cu) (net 6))
 (segment (start 139.05992 73.20026) (end 137.48766 73.20026) (width 0.25) (layer F.Cu) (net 6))
 (segment (start 140.615545 72.123999) (end 141.668946 73.1774) (width 0.25) (layer B.Cu) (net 6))
 (segment (start 136.411399 72.123999) (end 140.615545 72.123999) (width 0.25) (layer B.Cu) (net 6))
 (segment (start 135.6614 71.374) (end 136.411399 72.123999) (width 0.25) (layer B.Cu) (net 6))
 (segment (start 163.487799 67.780599) (end 162.7378 67.0306) (width 0.25) (layer B.Cu) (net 6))
 (segment (start 163.962001 68.254801) (end 163.487799 67.780599) (width 0.25) (layer B.Cu) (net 6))
 (segment (start 161.043402 73.1774) (end 163.962001 70.258801) (width 0.25) (layer B.Cu) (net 6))
 (segment (start 163.962001 70.258801) (end 163.962001 68.254801) (width 0.25) (layer B.Cu) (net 6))
 (segment (start 141.668946 73.1774) (end 161.043402 73.1774) (width 0.25) (layer B.Cu) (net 6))
 (segment (start 154.20594 67.056) (end 154.18054 67.0814) (width 0.25) (layer F.Cu) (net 5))
 (segment (start 156.845 67.056) (end 154.20594 67.056) (width 0.25) (layer F.Cu) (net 5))
 (segment (start 139.86002 72.10298) (end 141.6304 70.3326) (width 0.25) (layer F.Cu) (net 5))
 (segment (start 139.86002 73.1266) (end 139.86002 72.10298) (width 0.25) (layer F.Cu) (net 5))
 (segment (start 157.594999 67.805999) (end 156.845 67.056) (width 0.25) (layer B.Cu) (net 5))
 (segment (start 158.069201 68.280201) (end 157.594999 67.805999) (width 0.25) (layer B.Cu) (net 5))
 (segment (start 158.069201 70.258801) (end 158.069201 68.280201) (width 0.25) (layer B.Cu) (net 5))
 (segment (start 157.137191 71.190811) (end 158.069201 70.258801) (width 0.25) (layer B.Cu) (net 5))
 (segment (start 147.302357 71.190811) (end 157.137191 71.190811) (width 0.25) (layer B.Cu) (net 5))
 (segment (start 145.694147 69.582601) (end 147.302357 71.190811) (width 0.25) (layer B.Cu) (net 5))
 (segment (start 142.380399 69.582601) (end 145.694147 69.582601) (width 0.25) (layer B.Cu) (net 5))
 (segment (start 141.6304 70.3326) (end 142.380399 69.582601) (width 0.25) (layer B.Cu) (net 5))
 (segment (start 151.735529 62.083919) (end 151.735529 65.908929) (width 0.25) (layer F.Cu) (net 3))
 (segment (start 142.25778 64.5414) (end 142.25778 63.347934) (width 0.25) (layer F.Cu) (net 3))
 (segment (start 143.521795 62.083919) (end 151.735529 62.083919) (width 0.25) (layer F.Cu) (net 3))
 (segment (start 142.25778 63.347934) (end 143.521795 62.083919) (width 0.25) (layer F.Cu) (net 3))
 (segment (start 156.105069 65.908929) (end 151.735529 65.908929) (width 0.25) (layer F.Cu) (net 3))
 (segment (start 157.472598 64.5414) (end 156.105069 65.908929) (width 0.25) (layer F.Cu) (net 3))
 (segment (start 159.639 64.5414) (end 157.472598 64.5414) (width 0.25) (layer F.Cu) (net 3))
 (segment (start 140.66012 63.6564) (end 140.66012 64.5414) (width 0.25) (layer F.Cu) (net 2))
 (segment (start 140.66012 63.10709) (end 140.66012 63.6564) (width 0.25) (layer F.Cu) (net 2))
 (segment (start 159.080401 58.592799) (end 145.174411 58.592799) (width 0.25) (layer F.Cu) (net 2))
 (segment (start 161.434001 63.056401) (end 161.434001 60.946399) (width 0.25) (layer F.Cu) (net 2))
 (segment (start 161.329001 63.161401) (end 161.434001 63.056401) (width 0.25) (layer F.Cu) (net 2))
 (segment (start 161.434001 60.946399) (end 159.080401 58.592799) (width 0.25) (layer F.Cu) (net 2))
 (segment (start 157.878251 63.161401) (end 161.329001 63.161401) (width 0.25) (layer F.Cu) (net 2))
 (segment (start 156.498252 64.5414) (end 157.878251 63.161401) (width 0.25) (layer F.Cu) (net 2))
 (segment (start 145.174411 58.592799) (end 140.66012 63.10709) (width 0.25) (layer F.Cu) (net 2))
 (segment (start 154.18054 64.5414) (end 156.498252 64.5414) (width 0.25) (layer F.Cu) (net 2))
 (segment (start 152.385539 63.133461) (end 152.413479 63.161401) (width 0.25) (layer F.Cu) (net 1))
 (segment (start 143.252553 61.433909) (end 152.385539 61.433909) (width 0.25) (layer F.Cu) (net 1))
 (segment (start 141.46022 63.226242) (end 143.252553 61.433909) (width 0.25) (layer F.Cu) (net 1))
 (segment (start 152.385539 61.433909) (end 152.385539 63.133461) (width 0.25) (layer F.Cu) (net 1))
 (segment (start 141.46022 64.5414) (end 141.46022 63.226242) (width 0.25) (layer F.Cu) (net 1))
 (segment (start 156.958999 63.161401) (end 152.413479 63.161401) (width 0.25) (layer F.Cu) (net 1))
 (segment (start 158.119 62.0014) (end 156.958999 63.161401) (width 0.25) (layer F.Cu) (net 1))
 (segment (start 159.639 62.0014) (end 158.119 62.0014) (width 0.25) (layer F.Cu) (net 1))
 (segment (start 138.63212 64.46774) (end 139.05992 64.46774) (width 0.25) (layer F.Cu) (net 19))
 (segment (start 136.793008 64.46774) (end 138.63212 64.46774) (width 0.25) (layer F.Cu) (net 19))
 (segment (start 133.806747 67.454001) (end 136.793008 64.46774) (width 0.25) (layer F.Cu) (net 19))
 (segment (start 130.355997 67.454001) (end 133.806747 67.454001) (width 0.25) (layer F.Cu) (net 19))
 (segment (start 130.030999 67.778999) (end 130.355997 67.454001) (width 0.25) (layer F.Cu) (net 19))
 (segment (start 130.030999 70.213999) (end 130.030999 67.778999) (width 0.25) (layer F.Cu) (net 19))
 (segment (start 131.191 71.374) (end 130.030999 70.213999) (width 0.25) (layer F.Cu) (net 19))
 (segment (start 131.826 71.374) (end 131.191 71.374) (width 0.25) (layer F.Cu) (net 19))
 (segment (start 131.826 68.834) (end 132.461 68.834) (width 0.25) (layer F.Cu) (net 20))
 (segment (start 136.68394 66.03492) (end 137.49274 66.03492) (width 0.25) (layer F.Cu) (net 20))
 (segment (start 133.346 68.834) (end 136.14508 66.03492) (width 0.25) (layer F.Cu) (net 20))
 (segment (start 136.14508 66.03492) (end 136.68394 66.03492) (width 0.25) (layer F.Cu) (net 20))
 (segment (start 131.826 68.834) (end 133.346 68.834) (width 0.25) (layer F.Cu) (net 20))
 (segment (start 127.00254 68.834) (end 126.36754 68.834) (width 0.25) (layer F.Cu) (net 18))
 (segment (start 128.730979 67.105561) (end 127.00254 68.834) (width 0.25) (layer F.Cu) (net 18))
 (segment (start 128.730979 66.539019) (end 128.730979 67.105561) (width 0.25) (layer F.Cu) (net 18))
 (segment (start 131.886059 63.383939) (end 128.730979 66.539019) (width 0.25) (layer F.Cu) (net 18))
 (segment (start 139.86002 64.5414) (end 139.86002 63.586238) (width 0.25) (layer F.Cu) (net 18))
 (segment (start 139.86002 63.586238) (end 139.657721 63.383939) (width 0.25) (layer F.Cu) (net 18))
 (segment (start 139.657721 63.383939) (end 131.886059 63.383939) (width 0.25) (layer F.Cu) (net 18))
 (segment (start 142.25778 73.71842) (end 142.25778 73.1266) (width 0.25) (layer F.Cu) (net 26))
 (segment (start 142.25778 74.0116) (end 142.25778 73.1266) (width 0.25) (layer F.Cu) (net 26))
 (segment (start 142.25778 74.083032) (end 142.25778 74.0116) (width 0.25) (layer F.Cu) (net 26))
 (segment (start 142.054211 74.286601) (end 142.25778 74.083032) (width 0.25) (layer F.Cu) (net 26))
 (segment (start 131.888599 74.286601) (end 142.054211 74.286601) (width 0.25) (layer F.Cu) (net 26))
 (segment (start 129.380989 71.778991) (end 131.888599 74.286601) (width 0.25) (layer F.Cu) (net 26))
 (segment (start 129.380989 67.219011) (end 129.380989 71.778991) (width 0.25) (layer F.Cu) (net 26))
 (segment (start 130.306 66.294) (end 129.380989 67.219011) (width 0.25) (layer F.Cu) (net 26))
 (segment (start 131.826 66.294) (end 130.306 66.294) (width 0.25) (layer F.Cu) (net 26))
 (segment (start 136.12114 75.66914) (end 136.144 75.692) (width 0.25) (layer F.Cu) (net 30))
 (segment (start 132.334 75.66914) (end 136.12114 75.66914) (width 0.25) (layer F.Cu) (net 30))
 (segment (start 143.51 76.2) (end 140.589 76.2) (width 0.25) (layer F.Cu) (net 29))
 (segment (start 140.56868 79.0194) (end 140.589 79.03972) (width 0.25) (layer F.Cu) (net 24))
 (segment (start 143.18594 71.12) (end 144.2466 71.12) (width 0.25) (layer F.Cu) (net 24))
 (segment (start 142.698339 71.607601) (end 143.18594 71.12) (width 0.25) (layer F.Cu) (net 24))
 (segment (start 141.294119 71.607601) (end 142.698339 71.607601) (width 0.25) (layer F.Cu) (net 24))
 (segment (start 140.66012 72.2416) (end 141.294119 71.607601) (width 0.25) (layer F.Cu) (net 24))
 (segment (start 140.66012 73.1266) (end 140.66012 72.2416) (width 0.25) (layer F.Cu) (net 24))
 (segment (start 138.39952 79.03972) (end 138.3792 79.0194) (width 0.25) (layer F.Cu) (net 24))
 (segment (start 140.589 79.03972) (end 138.39952 79.03972) (width 0.25) (layer F.Cu) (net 24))
 (segment (start 138.3792 79.0194) (end 159.1564 79.0194) (width 0.25) (layer B.Cu) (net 24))
 (segment (start 159.1564 79.0194) (end 165.0746 73.1012) (width 0.25) (layer B.Cu) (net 24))
 (segment (start 144.996599 71.869999) (end 144.2466 71.12) (width 0.25) (layer B.Cu) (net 24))
 (segment (start 157.377255 71.869999) (end 144.996599 71.869999) (width 0.25) (layer B.Cu) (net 24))
 (segment (start 158.719211 70.528043) (end 157.377255 71.869999) (width 0.25) (layer B.Cu) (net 24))
 (segment (start 158.719211 69.162187) (end 158.719211 70.528043) (width 0.25) (layer B.Cu) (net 24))
 (segment (start 162.125799 65.755599) (end 158.719211 69.162187) (width 0.25) (layer B.Cu) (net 24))
 (segment (start 165.0746 67.480398) (end 163.349801 65.755599) (width 0.25) (layer B.Cu) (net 24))
 (segment (start 163.349801 65.755599) (end 162.125799 65.755599) (width 0.25) (layer B.Cu) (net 24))
 (segment (start 165.0746 73.1012) (end 165.0746 67.480398) (width 0.25) (layer B.Cu) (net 24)))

